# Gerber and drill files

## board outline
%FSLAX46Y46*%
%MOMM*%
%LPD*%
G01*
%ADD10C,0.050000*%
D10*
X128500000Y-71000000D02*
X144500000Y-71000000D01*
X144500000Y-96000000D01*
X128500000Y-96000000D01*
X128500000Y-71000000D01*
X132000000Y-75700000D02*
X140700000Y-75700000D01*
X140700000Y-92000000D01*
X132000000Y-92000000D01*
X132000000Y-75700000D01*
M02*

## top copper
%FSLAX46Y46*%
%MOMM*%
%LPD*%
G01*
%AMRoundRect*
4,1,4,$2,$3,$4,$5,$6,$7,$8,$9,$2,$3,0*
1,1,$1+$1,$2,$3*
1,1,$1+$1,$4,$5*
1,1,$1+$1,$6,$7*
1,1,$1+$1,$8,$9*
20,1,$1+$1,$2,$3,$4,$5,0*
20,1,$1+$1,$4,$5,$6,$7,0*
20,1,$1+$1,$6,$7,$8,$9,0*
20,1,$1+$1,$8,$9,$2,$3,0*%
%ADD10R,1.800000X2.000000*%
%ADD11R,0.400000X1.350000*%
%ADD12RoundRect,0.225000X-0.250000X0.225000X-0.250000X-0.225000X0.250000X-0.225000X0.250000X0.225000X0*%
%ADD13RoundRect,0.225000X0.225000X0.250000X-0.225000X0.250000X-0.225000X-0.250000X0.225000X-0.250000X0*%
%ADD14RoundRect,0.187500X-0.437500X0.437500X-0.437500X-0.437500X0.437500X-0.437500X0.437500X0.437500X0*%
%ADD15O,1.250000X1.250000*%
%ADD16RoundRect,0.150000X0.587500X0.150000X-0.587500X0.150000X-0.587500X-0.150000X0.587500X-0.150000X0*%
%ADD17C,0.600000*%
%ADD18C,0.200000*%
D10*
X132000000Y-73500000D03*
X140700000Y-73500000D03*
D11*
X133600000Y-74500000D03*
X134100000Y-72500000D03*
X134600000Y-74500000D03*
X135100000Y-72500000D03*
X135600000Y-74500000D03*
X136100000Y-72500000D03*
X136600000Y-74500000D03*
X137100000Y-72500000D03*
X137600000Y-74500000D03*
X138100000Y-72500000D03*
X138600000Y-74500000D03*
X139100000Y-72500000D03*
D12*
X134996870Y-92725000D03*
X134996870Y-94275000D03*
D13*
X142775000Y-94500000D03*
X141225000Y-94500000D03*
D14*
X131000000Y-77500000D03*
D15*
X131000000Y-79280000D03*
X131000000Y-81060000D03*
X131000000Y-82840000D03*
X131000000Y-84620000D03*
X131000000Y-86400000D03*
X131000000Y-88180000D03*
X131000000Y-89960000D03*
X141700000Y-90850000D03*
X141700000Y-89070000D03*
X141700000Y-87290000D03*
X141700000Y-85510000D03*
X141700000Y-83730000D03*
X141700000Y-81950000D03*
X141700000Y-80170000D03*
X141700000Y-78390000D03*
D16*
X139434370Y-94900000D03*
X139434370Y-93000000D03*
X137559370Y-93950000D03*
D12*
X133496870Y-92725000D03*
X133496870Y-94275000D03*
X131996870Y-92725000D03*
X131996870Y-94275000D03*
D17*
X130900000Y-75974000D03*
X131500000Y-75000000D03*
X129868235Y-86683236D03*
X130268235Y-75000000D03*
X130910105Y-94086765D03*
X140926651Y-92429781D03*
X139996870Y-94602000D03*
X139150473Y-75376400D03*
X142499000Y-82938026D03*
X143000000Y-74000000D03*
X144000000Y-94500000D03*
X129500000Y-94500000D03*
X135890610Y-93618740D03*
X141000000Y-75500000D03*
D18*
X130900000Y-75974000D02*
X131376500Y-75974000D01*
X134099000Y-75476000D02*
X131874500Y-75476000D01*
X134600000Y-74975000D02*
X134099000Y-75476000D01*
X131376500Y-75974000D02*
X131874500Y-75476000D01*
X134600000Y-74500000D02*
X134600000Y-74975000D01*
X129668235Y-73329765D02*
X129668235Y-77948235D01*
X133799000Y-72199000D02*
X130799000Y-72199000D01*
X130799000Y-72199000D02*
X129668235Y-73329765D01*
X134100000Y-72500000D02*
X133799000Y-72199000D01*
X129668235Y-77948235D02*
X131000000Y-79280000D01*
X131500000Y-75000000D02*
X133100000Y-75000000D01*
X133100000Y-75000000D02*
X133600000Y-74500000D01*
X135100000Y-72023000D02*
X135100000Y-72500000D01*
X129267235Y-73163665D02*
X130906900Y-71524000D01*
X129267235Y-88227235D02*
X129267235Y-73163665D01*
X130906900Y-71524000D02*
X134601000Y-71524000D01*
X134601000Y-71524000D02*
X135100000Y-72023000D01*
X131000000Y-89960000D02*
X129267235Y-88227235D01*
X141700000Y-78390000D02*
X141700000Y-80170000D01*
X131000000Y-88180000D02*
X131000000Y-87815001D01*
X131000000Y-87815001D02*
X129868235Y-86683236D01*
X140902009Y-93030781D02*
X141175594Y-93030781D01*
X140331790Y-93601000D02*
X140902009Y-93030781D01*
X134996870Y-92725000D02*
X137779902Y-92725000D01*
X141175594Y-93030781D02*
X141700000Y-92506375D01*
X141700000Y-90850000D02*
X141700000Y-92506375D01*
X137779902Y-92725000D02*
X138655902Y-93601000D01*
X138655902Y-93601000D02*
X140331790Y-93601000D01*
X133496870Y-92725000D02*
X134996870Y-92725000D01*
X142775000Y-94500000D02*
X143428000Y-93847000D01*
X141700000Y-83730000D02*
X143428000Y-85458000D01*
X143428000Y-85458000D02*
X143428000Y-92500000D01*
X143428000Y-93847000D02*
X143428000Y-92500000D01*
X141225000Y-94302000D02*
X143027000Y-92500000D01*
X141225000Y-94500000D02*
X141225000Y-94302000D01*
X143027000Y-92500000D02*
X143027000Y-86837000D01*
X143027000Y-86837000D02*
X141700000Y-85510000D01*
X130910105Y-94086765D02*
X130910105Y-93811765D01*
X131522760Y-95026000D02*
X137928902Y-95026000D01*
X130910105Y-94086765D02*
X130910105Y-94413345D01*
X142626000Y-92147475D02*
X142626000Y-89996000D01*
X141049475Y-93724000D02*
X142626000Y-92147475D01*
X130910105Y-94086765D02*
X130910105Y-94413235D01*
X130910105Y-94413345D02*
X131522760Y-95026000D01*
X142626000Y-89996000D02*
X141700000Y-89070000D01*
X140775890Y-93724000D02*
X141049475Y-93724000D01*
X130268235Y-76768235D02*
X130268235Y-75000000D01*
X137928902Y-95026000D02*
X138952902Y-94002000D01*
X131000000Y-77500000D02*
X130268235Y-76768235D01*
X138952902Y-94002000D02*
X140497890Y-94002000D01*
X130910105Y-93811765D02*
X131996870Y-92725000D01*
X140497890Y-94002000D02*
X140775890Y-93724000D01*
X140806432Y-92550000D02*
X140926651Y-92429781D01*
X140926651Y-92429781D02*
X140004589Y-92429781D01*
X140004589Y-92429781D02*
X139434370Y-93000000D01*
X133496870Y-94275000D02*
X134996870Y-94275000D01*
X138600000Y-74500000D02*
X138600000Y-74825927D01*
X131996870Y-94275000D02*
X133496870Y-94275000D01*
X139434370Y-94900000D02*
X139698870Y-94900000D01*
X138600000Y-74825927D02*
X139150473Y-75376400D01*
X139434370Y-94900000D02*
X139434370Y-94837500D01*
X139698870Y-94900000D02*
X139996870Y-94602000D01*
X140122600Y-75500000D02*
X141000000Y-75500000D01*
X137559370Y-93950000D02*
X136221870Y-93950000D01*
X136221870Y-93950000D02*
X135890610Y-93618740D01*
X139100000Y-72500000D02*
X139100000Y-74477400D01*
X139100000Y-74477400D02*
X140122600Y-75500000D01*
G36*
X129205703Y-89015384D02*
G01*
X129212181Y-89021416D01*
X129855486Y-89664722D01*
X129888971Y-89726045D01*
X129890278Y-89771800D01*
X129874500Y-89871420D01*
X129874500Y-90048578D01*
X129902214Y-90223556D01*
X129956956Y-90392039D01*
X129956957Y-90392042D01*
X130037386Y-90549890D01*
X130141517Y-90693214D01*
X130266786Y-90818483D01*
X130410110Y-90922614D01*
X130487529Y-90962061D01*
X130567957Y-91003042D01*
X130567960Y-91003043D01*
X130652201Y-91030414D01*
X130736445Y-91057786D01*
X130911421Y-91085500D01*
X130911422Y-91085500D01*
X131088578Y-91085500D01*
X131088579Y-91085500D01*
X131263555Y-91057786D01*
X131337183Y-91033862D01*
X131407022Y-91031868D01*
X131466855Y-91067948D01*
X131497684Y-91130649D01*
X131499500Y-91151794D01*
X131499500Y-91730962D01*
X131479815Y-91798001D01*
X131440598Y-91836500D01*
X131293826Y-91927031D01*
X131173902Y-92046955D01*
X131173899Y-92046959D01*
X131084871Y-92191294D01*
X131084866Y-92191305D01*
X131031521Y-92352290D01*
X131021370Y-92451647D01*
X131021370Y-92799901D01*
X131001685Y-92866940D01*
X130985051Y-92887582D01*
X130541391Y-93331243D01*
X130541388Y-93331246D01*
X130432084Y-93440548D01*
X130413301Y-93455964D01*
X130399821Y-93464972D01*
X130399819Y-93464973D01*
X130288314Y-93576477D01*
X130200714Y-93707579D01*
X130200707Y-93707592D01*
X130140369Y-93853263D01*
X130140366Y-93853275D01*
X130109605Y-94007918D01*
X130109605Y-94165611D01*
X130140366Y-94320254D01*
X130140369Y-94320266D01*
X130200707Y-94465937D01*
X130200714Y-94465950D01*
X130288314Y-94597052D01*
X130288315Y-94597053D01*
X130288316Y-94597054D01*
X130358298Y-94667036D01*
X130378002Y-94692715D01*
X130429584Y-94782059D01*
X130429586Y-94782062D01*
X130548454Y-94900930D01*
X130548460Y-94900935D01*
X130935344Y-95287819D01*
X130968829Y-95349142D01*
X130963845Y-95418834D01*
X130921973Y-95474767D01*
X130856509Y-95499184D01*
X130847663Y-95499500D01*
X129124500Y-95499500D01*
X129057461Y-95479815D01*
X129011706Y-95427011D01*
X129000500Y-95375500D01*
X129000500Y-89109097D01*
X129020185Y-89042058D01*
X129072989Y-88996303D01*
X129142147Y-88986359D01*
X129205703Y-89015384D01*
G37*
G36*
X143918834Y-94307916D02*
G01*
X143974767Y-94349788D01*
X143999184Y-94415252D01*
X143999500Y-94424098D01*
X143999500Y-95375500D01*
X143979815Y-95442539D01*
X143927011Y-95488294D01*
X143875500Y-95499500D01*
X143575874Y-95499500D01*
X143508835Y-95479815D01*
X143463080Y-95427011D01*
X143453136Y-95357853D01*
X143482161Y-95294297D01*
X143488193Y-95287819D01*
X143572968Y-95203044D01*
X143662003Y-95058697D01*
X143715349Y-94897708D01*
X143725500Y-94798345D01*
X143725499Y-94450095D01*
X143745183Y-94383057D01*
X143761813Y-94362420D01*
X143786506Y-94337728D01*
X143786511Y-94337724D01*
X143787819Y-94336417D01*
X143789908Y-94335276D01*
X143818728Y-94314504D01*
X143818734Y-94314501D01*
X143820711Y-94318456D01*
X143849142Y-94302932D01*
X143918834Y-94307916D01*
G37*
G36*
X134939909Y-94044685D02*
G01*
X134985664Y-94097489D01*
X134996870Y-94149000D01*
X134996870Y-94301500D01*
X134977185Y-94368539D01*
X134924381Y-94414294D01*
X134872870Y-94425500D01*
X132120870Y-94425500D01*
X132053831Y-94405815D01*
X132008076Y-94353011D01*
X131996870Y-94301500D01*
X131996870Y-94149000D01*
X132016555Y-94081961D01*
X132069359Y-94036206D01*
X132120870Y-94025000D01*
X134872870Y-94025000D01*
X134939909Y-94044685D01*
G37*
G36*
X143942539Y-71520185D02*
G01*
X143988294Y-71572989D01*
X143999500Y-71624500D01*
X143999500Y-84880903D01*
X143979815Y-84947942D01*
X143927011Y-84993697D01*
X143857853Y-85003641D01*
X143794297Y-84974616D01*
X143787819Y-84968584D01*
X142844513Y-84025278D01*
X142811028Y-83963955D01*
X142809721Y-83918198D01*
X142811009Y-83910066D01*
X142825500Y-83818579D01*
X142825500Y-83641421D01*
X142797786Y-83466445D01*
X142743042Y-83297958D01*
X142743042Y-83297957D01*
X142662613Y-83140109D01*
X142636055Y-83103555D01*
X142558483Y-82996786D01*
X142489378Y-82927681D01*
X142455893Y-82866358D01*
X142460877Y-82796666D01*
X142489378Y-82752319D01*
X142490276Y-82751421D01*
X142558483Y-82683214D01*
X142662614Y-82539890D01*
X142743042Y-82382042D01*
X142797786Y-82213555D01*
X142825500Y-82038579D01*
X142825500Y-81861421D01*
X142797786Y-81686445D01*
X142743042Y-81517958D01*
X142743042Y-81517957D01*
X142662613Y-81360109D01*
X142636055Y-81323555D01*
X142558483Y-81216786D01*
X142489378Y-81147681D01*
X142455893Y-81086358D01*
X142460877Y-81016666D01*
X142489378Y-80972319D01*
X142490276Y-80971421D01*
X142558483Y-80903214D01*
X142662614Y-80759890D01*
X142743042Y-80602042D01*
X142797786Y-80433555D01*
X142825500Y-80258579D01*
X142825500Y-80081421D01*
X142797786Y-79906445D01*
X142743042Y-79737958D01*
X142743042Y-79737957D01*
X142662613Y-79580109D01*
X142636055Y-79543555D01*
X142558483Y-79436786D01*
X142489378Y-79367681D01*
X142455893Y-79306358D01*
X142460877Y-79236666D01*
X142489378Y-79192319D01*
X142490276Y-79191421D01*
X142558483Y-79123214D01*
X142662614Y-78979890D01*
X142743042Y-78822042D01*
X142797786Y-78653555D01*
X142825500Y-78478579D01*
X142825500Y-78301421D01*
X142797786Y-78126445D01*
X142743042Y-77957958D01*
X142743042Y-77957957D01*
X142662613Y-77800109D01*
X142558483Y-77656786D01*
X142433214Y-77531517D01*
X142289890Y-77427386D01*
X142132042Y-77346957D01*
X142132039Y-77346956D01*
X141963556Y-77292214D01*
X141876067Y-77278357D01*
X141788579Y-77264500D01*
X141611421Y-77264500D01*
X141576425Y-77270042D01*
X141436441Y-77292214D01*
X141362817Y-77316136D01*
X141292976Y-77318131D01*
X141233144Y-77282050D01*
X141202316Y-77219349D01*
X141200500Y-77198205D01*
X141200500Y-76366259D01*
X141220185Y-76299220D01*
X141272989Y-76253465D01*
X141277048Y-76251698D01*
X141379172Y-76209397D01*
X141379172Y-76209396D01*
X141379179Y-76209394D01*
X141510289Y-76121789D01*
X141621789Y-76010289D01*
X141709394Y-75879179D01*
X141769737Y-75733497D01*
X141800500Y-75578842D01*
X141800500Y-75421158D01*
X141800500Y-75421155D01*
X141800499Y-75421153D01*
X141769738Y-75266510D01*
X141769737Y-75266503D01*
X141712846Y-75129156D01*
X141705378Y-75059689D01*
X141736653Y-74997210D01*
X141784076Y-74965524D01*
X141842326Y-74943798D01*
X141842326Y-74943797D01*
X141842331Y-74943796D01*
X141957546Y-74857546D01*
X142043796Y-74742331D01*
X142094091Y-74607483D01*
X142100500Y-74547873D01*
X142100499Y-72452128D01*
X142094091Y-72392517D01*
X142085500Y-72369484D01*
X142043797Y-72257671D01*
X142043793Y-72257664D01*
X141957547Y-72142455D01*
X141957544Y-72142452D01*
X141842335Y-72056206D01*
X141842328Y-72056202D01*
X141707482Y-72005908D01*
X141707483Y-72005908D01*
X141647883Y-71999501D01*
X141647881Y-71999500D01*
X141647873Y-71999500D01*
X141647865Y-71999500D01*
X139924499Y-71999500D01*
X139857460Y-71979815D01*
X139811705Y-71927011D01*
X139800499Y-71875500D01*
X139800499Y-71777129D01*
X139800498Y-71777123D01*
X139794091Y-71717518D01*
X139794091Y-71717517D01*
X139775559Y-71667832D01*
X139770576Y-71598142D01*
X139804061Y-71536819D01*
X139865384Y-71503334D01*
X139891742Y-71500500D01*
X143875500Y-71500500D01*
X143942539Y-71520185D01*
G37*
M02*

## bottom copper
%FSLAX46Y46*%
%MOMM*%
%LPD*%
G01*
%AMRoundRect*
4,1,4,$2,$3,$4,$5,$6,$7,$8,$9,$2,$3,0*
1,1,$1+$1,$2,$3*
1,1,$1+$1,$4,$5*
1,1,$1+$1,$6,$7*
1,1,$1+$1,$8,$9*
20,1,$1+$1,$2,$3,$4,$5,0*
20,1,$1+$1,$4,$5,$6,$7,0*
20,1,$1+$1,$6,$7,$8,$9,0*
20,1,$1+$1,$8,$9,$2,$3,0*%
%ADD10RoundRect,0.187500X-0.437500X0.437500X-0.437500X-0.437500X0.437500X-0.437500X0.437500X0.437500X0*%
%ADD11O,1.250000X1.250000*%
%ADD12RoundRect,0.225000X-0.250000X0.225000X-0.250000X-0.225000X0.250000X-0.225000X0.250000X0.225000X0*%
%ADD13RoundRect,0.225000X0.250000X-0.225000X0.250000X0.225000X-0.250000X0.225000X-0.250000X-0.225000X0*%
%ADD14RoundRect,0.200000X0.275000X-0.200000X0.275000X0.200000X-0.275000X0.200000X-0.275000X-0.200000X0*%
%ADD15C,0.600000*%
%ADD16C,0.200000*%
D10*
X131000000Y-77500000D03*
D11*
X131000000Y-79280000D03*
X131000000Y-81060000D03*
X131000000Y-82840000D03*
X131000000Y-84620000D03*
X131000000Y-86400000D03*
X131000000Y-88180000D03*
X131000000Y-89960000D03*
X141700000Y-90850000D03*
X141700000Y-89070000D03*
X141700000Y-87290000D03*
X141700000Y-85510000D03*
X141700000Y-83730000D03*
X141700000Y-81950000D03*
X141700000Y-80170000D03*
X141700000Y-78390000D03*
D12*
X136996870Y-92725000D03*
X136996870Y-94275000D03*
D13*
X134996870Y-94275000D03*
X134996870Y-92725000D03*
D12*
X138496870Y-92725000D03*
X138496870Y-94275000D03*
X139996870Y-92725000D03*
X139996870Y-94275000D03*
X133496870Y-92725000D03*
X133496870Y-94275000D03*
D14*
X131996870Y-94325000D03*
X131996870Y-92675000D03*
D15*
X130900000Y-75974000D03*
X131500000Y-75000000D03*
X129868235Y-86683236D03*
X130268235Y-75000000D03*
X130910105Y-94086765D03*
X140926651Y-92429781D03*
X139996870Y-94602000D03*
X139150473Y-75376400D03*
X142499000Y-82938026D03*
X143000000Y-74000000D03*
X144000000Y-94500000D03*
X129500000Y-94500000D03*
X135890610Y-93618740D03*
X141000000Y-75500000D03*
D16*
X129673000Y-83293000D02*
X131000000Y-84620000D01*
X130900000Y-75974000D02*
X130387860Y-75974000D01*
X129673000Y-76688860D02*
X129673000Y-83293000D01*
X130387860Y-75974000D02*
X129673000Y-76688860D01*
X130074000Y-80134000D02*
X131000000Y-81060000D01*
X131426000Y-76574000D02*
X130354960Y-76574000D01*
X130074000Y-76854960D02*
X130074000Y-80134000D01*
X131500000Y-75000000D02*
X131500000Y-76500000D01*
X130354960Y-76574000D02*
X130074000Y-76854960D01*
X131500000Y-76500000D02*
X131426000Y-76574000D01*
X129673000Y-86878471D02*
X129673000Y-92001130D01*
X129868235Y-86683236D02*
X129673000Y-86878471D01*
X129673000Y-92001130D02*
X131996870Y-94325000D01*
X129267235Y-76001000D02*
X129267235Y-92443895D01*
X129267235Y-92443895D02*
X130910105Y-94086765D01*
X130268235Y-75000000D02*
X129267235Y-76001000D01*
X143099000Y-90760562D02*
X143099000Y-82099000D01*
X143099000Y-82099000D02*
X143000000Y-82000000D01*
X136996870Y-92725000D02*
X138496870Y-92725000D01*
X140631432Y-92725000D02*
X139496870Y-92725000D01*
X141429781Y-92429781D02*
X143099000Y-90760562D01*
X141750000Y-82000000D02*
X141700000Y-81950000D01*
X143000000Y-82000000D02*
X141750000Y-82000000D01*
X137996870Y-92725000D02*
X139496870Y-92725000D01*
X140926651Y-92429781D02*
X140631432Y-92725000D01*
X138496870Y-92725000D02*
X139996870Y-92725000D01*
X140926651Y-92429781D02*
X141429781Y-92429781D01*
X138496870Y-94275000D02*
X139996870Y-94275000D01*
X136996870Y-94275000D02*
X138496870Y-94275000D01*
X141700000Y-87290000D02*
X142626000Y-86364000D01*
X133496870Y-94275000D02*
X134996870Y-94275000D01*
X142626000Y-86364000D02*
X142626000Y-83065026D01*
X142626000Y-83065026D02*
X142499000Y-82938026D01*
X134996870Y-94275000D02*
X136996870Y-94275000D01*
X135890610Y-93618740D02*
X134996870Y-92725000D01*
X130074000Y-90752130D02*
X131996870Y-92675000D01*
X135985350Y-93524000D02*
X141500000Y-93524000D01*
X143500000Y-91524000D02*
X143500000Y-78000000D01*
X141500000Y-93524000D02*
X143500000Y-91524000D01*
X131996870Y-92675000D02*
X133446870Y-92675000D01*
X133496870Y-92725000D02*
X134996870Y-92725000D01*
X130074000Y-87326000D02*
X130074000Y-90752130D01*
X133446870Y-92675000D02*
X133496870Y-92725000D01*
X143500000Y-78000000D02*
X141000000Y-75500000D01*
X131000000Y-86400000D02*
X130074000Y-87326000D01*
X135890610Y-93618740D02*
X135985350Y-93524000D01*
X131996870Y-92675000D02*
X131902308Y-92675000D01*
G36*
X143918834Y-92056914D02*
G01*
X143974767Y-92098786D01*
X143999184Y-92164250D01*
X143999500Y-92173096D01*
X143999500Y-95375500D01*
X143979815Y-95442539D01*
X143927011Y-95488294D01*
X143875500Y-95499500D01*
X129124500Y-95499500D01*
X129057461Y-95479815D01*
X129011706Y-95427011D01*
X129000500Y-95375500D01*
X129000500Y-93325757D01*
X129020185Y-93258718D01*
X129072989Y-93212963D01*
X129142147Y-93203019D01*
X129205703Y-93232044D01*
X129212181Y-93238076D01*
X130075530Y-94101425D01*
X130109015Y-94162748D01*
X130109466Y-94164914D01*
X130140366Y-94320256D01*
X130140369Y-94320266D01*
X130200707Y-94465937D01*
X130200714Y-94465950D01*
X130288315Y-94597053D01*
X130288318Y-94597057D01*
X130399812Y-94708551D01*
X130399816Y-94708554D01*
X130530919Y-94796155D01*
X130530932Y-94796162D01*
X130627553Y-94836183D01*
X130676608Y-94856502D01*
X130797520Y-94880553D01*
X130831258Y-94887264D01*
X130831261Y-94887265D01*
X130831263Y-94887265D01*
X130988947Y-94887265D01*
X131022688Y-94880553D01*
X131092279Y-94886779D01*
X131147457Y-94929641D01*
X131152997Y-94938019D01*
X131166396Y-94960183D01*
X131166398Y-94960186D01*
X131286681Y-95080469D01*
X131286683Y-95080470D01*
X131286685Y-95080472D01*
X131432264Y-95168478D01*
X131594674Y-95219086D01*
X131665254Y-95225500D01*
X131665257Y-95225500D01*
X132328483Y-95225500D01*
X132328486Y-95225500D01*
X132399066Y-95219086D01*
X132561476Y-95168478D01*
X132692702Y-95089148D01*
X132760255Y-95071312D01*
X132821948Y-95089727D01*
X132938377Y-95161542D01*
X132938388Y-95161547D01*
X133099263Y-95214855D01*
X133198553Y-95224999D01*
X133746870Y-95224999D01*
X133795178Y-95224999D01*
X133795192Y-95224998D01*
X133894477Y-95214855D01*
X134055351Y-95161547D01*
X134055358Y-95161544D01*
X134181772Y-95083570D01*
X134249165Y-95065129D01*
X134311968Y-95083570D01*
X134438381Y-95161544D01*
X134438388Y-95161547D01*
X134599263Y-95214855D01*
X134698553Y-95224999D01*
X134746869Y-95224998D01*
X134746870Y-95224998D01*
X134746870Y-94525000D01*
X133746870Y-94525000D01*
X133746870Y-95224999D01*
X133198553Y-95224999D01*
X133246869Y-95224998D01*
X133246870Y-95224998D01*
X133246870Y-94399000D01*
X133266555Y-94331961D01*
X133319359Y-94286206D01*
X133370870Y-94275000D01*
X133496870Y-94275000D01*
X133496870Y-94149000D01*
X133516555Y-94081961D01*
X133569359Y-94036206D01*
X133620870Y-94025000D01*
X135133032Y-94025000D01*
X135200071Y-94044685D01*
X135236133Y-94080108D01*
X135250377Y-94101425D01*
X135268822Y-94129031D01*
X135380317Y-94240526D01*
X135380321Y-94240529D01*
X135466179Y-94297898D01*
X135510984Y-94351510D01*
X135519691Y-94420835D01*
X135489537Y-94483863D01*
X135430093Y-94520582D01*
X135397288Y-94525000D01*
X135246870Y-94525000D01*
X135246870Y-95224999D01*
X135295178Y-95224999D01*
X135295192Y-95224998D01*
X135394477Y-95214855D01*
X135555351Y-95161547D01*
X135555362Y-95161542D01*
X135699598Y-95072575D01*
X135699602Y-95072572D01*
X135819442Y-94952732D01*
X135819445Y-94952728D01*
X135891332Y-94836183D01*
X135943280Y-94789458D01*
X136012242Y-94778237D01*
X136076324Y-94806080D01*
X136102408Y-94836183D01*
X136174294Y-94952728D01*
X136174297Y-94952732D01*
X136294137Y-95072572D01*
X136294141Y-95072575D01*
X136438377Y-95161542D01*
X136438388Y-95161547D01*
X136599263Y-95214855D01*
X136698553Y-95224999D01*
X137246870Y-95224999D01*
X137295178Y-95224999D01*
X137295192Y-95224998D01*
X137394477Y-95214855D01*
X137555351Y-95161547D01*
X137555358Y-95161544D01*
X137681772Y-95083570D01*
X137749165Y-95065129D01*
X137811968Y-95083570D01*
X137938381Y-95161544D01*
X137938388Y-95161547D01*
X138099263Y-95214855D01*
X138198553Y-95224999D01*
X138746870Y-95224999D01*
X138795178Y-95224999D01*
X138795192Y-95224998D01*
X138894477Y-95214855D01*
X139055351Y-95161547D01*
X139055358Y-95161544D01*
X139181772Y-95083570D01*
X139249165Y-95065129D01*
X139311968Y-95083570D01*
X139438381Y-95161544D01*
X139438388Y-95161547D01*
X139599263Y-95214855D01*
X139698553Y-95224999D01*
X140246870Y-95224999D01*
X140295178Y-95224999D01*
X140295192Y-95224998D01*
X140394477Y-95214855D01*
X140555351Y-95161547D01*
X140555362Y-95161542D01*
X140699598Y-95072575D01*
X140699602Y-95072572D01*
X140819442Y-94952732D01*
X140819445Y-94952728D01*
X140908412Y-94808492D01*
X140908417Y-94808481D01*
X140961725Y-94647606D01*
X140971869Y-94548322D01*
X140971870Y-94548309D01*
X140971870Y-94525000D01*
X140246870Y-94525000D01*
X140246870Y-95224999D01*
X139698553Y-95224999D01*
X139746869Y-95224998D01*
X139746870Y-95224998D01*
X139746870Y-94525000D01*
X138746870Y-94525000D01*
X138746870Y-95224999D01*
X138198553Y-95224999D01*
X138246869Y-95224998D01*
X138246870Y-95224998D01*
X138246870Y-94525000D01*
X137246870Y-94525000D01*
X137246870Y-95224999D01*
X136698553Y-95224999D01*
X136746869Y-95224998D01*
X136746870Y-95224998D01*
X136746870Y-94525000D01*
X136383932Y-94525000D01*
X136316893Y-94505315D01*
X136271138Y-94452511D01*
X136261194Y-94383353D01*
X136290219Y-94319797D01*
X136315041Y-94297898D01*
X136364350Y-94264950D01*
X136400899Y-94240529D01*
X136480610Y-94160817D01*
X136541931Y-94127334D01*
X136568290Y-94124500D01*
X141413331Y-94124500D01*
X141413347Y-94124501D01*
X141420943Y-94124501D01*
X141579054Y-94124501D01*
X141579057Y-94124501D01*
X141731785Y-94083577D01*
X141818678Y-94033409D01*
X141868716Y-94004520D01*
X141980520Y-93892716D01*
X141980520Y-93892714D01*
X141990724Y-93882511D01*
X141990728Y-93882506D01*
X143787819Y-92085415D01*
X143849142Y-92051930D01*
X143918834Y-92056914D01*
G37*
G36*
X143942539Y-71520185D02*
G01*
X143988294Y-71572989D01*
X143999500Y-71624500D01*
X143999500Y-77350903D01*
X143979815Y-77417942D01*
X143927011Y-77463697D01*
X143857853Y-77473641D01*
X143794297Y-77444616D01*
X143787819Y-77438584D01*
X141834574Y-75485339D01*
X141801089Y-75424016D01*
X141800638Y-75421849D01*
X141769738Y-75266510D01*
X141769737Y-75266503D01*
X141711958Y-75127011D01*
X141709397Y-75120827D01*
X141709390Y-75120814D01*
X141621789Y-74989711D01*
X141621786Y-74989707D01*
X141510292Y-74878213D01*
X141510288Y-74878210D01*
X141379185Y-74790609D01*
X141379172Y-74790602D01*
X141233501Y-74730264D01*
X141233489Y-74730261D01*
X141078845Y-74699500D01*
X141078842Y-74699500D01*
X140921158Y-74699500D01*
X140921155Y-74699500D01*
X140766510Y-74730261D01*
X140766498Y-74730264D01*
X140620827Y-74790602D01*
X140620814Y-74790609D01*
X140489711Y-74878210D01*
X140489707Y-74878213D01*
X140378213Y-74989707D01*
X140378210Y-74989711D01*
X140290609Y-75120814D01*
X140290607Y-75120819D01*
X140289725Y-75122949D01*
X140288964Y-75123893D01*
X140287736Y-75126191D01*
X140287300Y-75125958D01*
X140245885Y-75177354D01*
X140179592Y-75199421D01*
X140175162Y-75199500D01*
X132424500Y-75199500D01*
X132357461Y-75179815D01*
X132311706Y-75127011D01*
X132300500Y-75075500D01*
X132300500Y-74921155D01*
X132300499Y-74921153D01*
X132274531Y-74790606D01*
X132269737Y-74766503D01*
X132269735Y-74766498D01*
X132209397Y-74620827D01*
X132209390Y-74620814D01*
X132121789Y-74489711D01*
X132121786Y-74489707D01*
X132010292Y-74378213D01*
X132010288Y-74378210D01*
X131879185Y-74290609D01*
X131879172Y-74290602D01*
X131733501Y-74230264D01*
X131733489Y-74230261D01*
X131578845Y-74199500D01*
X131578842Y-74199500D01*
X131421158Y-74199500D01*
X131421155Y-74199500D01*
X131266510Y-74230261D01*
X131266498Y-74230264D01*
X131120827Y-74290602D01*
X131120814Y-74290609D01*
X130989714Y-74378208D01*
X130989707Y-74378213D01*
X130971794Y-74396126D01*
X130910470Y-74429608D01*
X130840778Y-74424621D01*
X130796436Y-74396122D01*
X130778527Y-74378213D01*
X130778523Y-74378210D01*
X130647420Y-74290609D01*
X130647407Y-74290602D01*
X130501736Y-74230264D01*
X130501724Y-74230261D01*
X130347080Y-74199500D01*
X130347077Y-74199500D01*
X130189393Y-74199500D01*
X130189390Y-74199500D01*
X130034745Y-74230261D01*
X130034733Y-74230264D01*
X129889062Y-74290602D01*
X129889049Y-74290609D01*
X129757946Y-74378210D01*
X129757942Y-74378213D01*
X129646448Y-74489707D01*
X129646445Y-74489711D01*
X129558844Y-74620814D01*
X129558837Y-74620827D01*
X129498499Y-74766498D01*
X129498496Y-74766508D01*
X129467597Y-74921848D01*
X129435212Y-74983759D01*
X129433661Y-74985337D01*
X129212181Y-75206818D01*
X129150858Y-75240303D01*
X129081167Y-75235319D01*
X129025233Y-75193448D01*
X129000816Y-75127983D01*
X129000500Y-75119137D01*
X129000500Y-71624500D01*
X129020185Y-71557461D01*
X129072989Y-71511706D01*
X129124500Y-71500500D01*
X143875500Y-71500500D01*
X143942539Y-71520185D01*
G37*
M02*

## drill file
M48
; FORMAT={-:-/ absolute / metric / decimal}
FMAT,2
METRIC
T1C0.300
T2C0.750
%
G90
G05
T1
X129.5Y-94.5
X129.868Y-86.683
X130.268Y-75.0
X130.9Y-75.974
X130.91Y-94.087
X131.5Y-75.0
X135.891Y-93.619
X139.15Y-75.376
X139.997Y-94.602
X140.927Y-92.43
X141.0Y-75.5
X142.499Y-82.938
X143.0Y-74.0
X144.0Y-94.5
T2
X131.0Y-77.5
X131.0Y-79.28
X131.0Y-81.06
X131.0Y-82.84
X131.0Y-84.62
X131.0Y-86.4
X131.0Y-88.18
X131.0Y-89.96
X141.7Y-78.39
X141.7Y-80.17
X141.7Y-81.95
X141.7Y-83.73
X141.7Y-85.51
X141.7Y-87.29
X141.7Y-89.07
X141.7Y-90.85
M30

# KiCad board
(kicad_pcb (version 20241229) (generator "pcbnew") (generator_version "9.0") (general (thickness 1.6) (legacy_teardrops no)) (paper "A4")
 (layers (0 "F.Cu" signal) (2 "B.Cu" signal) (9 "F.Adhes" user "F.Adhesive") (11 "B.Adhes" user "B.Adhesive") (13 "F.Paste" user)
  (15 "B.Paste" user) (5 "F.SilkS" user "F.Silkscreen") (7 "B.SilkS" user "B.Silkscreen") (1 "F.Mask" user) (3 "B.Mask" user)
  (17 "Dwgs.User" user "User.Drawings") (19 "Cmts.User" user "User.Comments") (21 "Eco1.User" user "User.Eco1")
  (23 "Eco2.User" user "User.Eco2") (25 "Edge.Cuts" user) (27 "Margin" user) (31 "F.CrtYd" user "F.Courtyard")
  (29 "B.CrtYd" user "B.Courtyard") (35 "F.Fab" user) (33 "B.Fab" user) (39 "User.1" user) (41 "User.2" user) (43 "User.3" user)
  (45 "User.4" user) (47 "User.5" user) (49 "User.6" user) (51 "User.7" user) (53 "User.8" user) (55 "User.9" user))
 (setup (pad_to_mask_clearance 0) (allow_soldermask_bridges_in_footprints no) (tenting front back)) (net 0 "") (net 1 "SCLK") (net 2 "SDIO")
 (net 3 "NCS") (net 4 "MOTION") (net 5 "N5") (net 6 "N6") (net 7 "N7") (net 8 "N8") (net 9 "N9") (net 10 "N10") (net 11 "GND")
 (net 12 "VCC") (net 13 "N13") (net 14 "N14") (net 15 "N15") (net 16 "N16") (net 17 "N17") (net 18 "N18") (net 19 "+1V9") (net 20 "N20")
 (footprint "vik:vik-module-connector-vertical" (layer "F.Cu") (at 136.35 73.5)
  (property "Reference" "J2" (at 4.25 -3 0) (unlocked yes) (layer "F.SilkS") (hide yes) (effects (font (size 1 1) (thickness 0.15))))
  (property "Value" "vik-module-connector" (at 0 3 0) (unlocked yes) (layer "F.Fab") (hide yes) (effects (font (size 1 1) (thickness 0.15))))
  (pad "" smd rect (at -4.35 0) (size 1.8 2) (layers "F.Cu" "F.Mask" "F.Paste") (thermal_bridge_angle 45))
  (pad "" smd rect (at 4.35 0) (size 1.8 2) (layers "F.Cu" "F.Mask" "F.Paste") (thermal_bridge_angle 45))
  (pad "1" smd rect (at -2.75 1) (size 0.4 1.35) (layers "F.Cu" "F.Mask" "F.Paste") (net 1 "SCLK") (thermal_bridge_angle 45))
  (pad "2" smd rect (at -2.25 -1) (size 0.4 1.35) (layers "F.Cu" "F.Mask" "F.Paste") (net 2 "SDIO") (thermal_bridge_angle 45))
  (pad "3" smd rect (at -1.75 1) (size 0.4 1.35) (layers "F.Cu" "F.Mask" "F.Paste") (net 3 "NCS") (thermal_bridge_angle 45))
  (pad "4" smd rect (at -1.25 -1) (size 0.4 1.35) (layers "F.Cu" "F.Mask" "F.Paste") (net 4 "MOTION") (thermal_bridge_angle 45))
  (pad "5" smd rect (at -0.75 1) (size 0.4 1.35) (layers "F.Cu" "F.Mask" "F.Paste") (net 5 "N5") (thermal_bridge_angle 45))
  (pad "6" smd rect (at -0.25 -1) (size 0.4 1.35) (layers "F.Cu" "F.Mask" "F.Paste") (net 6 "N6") (thermal_bridge_angle 45))
  (pad "7" smd rect (at 0.25 1) (size 0.4 1.35) (layers "F.Cu" "F.Mask" "F.Paste") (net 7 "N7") (thermal_bridge_angle 45))
  (pad "8" smd rect (at 0.75 -1) (size 0.4 1.35) (layers "F.Cu" "F.Mask" "F.Paste") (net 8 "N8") (thermal_bridge_angle 45))
  (pad "9" smd rect (at 1.25 1) (size 0.4 1.35) (layers "F.Cu" "F.Mask" "F.Paste") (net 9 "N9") (thermal_bridge_angle 45))
  (pad "10" smd rect (at 1.75 -1) (size 0.4 1.35) (layers "F.Cu" "F.Mask" "F.Paste") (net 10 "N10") (thermal_bridge_angle 45))
  (pad "11" smd rect (at 2.25 1) (size 0.4 1.35) (layers "F.Cu" "F.Mask" "F.Paste") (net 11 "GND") (thermal_bridge_angle 45))
  (pad "12" smd rect (at 2.75 -1) (size 0.4 1.35) (layers "F.Cu" "F.Mask" "F.Paste") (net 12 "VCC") (thermal_bridge_angle 45)))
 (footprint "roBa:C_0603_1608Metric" (layer "F.Cu") (at 134.99687 93.5 -90)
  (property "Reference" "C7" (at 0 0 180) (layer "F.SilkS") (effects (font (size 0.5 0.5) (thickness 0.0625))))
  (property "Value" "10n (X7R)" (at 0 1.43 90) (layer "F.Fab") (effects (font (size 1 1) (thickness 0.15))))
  (pad "1" smd roundrect (at -0.775 0 270) (size 0.9 0.95) (layers "F.Cu" "F.Mask" "F.Paste") (roundrect_rratio 0.25) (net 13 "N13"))
  (pad "2" smd roundrect (at 0.775 0 270) (size 0.9 0.95) (layers "F.Cu" "F.Mask" "F.Paste") (roundrect_rratio 0.25) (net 11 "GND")))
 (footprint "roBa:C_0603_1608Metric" (layer "F.Cu") (at 142 94.5 180)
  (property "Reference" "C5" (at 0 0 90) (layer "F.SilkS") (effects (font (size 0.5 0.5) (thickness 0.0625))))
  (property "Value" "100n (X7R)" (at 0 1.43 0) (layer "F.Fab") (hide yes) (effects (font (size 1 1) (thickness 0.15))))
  (pad "1" smd roundrect (at -0.775 0 180) (size 0.9 0.95) (layers "F.Cu" "F.Mask" "F.Paste") (roundrect_rratio 0.25) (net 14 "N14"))
  (pad "2" smd roundrect (at 0.775 0 180) (size 0.9 0.95) (layers "F.Cu" "F.Mask" "F.Paste") (roundrect_rratio 0.25) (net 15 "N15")))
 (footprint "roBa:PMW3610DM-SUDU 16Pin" (layer "F.Cu") (at 136.35 83.668 90)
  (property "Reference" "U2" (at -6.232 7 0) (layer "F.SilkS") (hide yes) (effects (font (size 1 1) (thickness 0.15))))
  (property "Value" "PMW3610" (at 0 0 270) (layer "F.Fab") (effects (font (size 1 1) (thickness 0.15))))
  (pad "1" thru_hole roundrect (at 6.168 -5.35 270) (size 1.25 1.25) (drill 0.75) (layers "*.Cu" "*.Mask") (remove_unused_layers no)
   (roundrect_rratio 0.15) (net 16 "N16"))
  (pad "2" thru_hole oval (at 4.388 -5.35 270) (size 1.25 1.25) (drill 0.75) (layers "*.Cu" "*.Mask") (remove_unused_layers no)
   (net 2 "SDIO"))
  (pad "3" thru_hole oval (at 2.608 -5.35 270) (size 1.25 1.25) (drill 0.75) (layers "*.Cu" "*.Mask") (remove_unused_layers no)
   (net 1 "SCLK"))
  (pad "4" thru_hole oval (at 0.828 -5.35 270) (size 1.25 1.25) (drill 0.75) (layers "*.Cu" "*.Mask") (remove_unused_layers no)
   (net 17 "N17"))
  (pad "5" thru_hole oval (at -0.952 -5.35 270) (size 1.25 1.25) (drill 0.75) (layers "*.Cu" "*.Mask") (remove_unused_layers no)
   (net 3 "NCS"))
  (pad "6" thru_hole oval (at -2.732 -5.35 270) (size 1.25 1.25) (drill 0.75) (layers "*.Cu" "*.Mask") (remove_unused_layers no)
   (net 12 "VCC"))
  (pad "7" thru_hole oval (at -4.512 -5.35 270) (size 1.25 1.25) (drill 0.75) (layers "*.Cu" "*.Mask") (remove_unused_layers no)
   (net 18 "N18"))
  (pad "8" thru_hole oval (at -6.292 -5.35 270) (size 1.25 1.25) (drill 0.75) (layers "*.Cu" "*.Mask") (remove_unused_layers no)
   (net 4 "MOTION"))
  (pad "9" thru_hole oval (at -7.182 5.35 270) (size 1.25 1.25) (drill 0.75) (layers "*.Cu" "*.Mask") (remove_unused_layers no)
   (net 13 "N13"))
  (pad "10" thru_hole oval (at -5.402 5.35 270) (size 1.25 1.25) (drill 0.75) (layers "*.Cu" "*.Mask") (remove_unused_layers no)
   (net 16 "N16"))
  (pad "11" thru_hole oval (at -3.622 5.35 270) (size 1.25 1.25) (drill 0.75) (layers "*.Cu" "*.Mask") (remove_unused_layers no)
   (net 11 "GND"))
  (pad "12" thru_hole oval (at -1.842 5.35 270) (size 1.25 1.25) (drill 0.75) (layers "*.Cu" "*.Mask") (remove_unused_layers no)
   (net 15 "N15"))
  (pad "13" thru_hole oval (at -0.062 5.35 270) (size 1.25 1.25) (drill 0.75) (layers "*.Cu" "*.Mask") (remove_unused_layers no)
   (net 14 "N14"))
  (pad "14" thru_hole oval (at 1.718 5.35 270) (size 1.25 1.25) (drill 0.75) (layers "*.Cu" "*.Mask") (remove_unused_layers no)
   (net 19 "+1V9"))
  (pad "15" thru_hole oval (at 3.498 5.35 270) (size 1.25 1.25) (drill 0.75) (layers "*.Cu" "*.Mask") (remove_unused_layers no)
   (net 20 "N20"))
  (pad "16" thru_hole oval (at 5.278 5.35 270) (size 1.25 1.25) (drill 0.75) (layers "*.Cu" "*.Mask") (remove_unused_layers no)
   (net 20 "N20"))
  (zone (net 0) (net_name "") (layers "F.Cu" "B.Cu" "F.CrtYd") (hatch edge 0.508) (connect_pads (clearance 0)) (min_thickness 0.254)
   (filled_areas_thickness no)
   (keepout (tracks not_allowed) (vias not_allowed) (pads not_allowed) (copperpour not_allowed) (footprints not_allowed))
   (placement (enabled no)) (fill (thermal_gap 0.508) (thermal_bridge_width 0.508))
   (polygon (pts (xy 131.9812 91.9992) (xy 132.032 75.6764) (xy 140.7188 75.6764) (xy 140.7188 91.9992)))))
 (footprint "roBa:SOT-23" (layer "F.Cu") (at 138.49687 93.95 180)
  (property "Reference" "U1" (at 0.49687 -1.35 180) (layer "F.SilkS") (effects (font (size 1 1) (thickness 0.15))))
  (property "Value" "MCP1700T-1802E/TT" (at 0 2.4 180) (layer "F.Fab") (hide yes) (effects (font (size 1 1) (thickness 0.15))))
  (pad "1" smd roundrect (at -0.9375 -0.95 180) (size 1.475 0.6) (layers "F.Cu" "F.Mask" "F.Paste") (roundrect_rratio 0.25) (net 11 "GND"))
  (pad "2" smd roundrect (at -0.9375 0.95 180) (size 1.475 0.6) (layers "F.Cu" "F.Mask" "F.Paste") (roundrect_rratio 0.25) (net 19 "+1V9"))
  (pad "3" smd roundrect (at 0.9375 0 180) (size 1.475 0.6) (layers "F.Cu" "F.Mask" "F.Paste") (roundrect_rratio 0.25) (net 12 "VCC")))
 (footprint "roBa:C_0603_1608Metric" (layer "F.Cu") (at 133.49687 93.5 -90)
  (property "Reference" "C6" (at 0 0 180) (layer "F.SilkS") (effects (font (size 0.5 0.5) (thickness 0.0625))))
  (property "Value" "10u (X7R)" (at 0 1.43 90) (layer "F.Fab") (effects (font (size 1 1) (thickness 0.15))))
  (pad "1" smd roundrect (at -0.775 0 270) (size 0.9 0.95) (layers "F.Cu" "F.Mask" "F.Paste") (roundrect_rratio 0.25) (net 13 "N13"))
  (pad "2" smd roundrect (at 0.775 0 270) (size 0.9 0.95) (layers "F.Cu" "F.Mask" "F.Paste") (roundrect_rratio 0.25) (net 11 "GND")))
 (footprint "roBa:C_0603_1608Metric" (layer "F.Cu") (at 131.99687 93.5 -90)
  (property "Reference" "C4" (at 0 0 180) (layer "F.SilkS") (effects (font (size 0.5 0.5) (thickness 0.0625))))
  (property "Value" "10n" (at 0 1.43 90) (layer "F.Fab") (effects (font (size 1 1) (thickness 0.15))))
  (pad "1" smd roundrect (at -0.775 0 270) (size 0.9 0.95) (layers "F.Cu" "F.Mask" "F.Paste") (roundrect_rratio 0.25) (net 16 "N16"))
  (pad "2" smd roundrect (at 0.775 0 270) (size 0.9 0.95) (layers "F.Cu" "F.Mask" "F.Paste") (roundrect_rratio 0.25) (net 11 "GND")))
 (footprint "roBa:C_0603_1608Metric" (layer "B.Cu") (at 136.99687 93.5 -90)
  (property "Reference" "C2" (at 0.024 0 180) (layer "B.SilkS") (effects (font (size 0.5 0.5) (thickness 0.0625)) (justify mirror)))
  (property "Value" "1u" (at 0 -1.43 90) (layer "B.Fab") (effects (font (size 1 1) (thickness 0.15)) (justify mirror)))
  (pad "1" smd roundrect (at -0.775 0 270) (size 0.9 0.95) (layers "B.Cu" "B.Mask" "B.Paste") (roundrect_rratio 0.25) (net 19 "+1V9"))
  (pad "2" smd roundrect (at 0.775 0 270) (size 0.9 0.95) (layers "B.Cu" "B.Mask" "B.Paste") (roundrect_rratio 0.25) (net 11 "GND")))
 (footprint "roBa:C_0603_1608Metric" (layer "B.Cu") (at 134.99687 93.5 90)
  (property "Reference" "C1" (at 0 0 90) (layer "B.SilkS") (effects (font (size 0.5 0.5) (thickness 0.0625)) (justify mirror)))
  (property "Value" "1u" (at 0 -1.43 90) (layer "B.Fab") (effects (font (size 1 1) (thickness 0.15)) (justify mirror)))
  (pad "1" smd roundrect (at -0.775 0 90) (size 0.9 0.95) (layers "B.Cu" "B.Mask" "B.Paste") (roundrect_rratio 0.25) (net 11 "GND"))
  (pad "2" smd roundrect (at 0.775 0 90) (size 0.9 0.95) (layers "B.Cu" "B.Mask" "B.Paste") (roundrect_rratio 0.25) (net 12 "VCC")))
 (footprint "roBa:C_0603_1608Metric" (layer "B.Cu") (at 138.49687 93.5 -90)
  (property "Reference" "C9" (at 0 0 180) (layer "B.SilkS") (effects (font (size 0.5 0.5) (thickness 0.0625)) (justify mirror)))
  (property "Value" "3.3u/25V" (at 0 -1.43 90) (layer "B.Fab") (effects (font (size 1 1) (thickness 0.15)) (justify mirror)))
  (pad "1" smd roundrect (at -0.775 0 270) (size 0.9 0.95) (layers "B.Cu" "B.Mask" "B.Paste") (roundrect_rratio 0.25) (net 19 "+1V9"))
  (pad "2" smd roundrect (at 0.775 0 270) (size 0.9 0.95) (layers "B.Cu" "B.Mask" "B.Paste") (roundrect_rratio 0.25) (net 11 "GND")))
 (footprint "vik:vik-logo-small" (layer "B.Cu") (at 142 74 90)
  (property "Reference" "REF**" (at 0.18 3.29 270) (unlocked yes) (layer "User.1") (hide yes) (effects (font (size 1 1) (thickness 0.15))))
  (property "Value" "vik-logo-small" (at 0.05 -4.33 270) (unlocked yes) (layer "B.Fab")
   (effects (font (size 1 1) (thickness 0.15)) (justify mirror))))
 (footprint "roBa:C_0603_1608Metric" (layer "B.Cu") (at 139.99687 93.5 -90)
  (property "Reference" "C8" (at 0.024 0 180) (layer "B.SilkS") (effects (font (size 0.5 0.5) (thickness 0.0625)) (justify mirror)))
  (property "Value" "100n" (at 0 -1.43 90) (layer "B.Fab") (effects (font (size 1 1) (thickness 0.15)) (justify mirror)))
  (pad "1" smd roundrect (at -0.775 0 270) (size 0.9 0.95) (layers "B.Cu" "B.Mask" "B.Paste") (roundrect_rratio 0.25) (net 19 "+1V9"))
  (pad "2" smd roundrect (at 0.775 0 270) (size 0.9 0.95) (layers "B.Cu" "B.Mask" "B.Paste") (roundrect_rratio 0.25) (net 11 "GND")))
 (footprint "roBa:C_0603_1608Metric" (layer "B.Cu") (at 133.49687 93.5 -90)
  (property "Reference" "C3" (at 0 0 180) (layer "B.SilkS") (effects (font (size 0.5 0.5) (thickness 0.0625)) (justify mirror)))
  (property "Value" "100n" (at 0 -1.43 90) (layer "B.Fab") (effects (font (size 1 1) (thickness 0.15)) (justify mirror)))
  (pad "1" smd roundrect (at -0.775 0 270) (size 0.9 0.95) (layers "B.Cu" "B.Mask" "B.Paste") (roundrect_rratio 0.25) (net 12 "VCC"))
  (pad "2" smd roundrect (at 0.775 0 270) (size 0.9 0.95) (layers "B.Cu" "B.Mask" "B.Paste") (roundrect_rratio 0.25) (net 11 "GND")))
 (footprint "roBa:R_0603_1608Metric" (layer "B.Cu") (at 131.99687 93.5 90)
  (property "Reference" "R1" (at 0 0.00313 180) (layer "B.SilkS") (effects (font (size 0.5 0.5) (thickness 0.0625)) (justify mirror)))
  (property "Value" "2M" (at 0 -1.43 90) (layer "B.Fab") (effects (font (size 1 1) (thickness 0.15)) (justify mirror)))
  (pad "1" smd roundrect (at -0.825 0 90) (size 0.8 0.95) (layers "B.Cu" "B.Mask" "B.Paste") (roundrect_rratio 0.25) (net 18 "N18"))
  (pad "2" smd roundrect (at 0.825 0 90) (size 0.8 0.95) (layers "B.Cu" "B.Mask" "B.Paste") (roundrect_rratio 0.25) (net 12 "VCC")))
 (gr_rect (start 128.5 71) (end 144.5 96) (stroke (width 0.05) (type default)) (fill no) (layer "Edge.Cuts"))
 (gr_rect (start 132 75.7) (end 140.7 92) (stroke (width 0.05) (type default)) (fill no) (layer "Edge.Cuts"))
 (segment (start 130.9 75.974) (end 131.3765 75.974) (width 0.2) (layer "F.Cu") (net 3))
 (segment (start 134.099 75.476) (end 131.8745 75.476) (width 0.2) (layer "F.Cu") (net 3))
 (segment (start 134.6 74.975) (end 134.099 75.476) (width 0.2) (layer "F.Cu") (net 3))
 (segment (start 131.3765 75.974) (end 131.8745 75.476) (width 0.2) (layer "F.Cu") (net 3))
 (segment (start 134.6 74.5) (end 134.6 74.975) (width 0.2) (layer "F.Cu") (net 3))
 (via (at 130.9 75.974) (size 0.6) (drill 0.3) (layers "F.Cu" "B.Cu") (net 3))
 (segment (start 129.673 83.293) (end 131 84.62) (width 0.2) (layer "B.Cu") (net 3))
 (segment (start 130.9 75.974) (end 130.38786 75.974) (width 0.2) (layer "B.Cu") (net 3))
 (segment (start 129.673 76.68886) (end 129.673 83.293) (width 0.2) (layer "B.Cu") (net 3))
 (segment (start 130.38786 75.974) (end 129.673 76.68886) (width 0.2) (layer "B.Cu") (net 3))
 (segment (start 129.668235 73.329765) (end 129.668235 77.948235) (width 0.2) (layer "F.Cu") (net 2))
 (segment (start 133.799 72.199) (end 130.799 72.199) (width 0.2) (layer "F.Cu") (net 2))
 (segment (start 130.799 72.199) (end 129.668235 73.329765) (width 0.2) (layer "F.Cu") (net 2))
 (segment (start 134.1 72.5) (end 133.799 72.199) (width 0.2) (layer "F.Cu") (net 2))
 (segment (start 129.668235 77.948235) (end 131 79.28) (width 0.2) (layer "F.Cu") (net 2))
 (segment (start 131.5 75) (end 133.1 75) (width 0.2) (layer "F.Cu") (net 1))
 (segment (start 133.1 75) (end 133.6 74.5) (width 0.2) (layer "F.Cu") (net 1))
 (via (at 131.5 75) (size 0.6) (drill 0.3) (layers "F.Cu" "B.Cu") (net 1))
 (segment (start 130.074 80.134) (end 131 81.06) (width 0.2) (layer "B.Cu") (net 1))
 (segment (start 131.426 76.574) (end 130.35496 76.574) (width 0.2) (layer "B.Cu") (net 1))
 (segment (start 130.074 76.85496) (end 130.074 80.134) (width 0.2) (layer "B.Cu") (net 1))
 (segment (start 131.5 75) (end 131.5 76.5) (width 0.2) (layer "B.Cu") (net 1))
 (segment (start 130.35496 76.574) (end 130.074 76.85496) (width 0.2) (layer "B.Cu") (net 1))
 (segment (start 131.5 76.5) (end 131.426 76.574) (width 0.2) (layer "B.Cu") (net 1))
 (segment (start 135.1 72.023) (end 135.1 72.5) (width 0.2) (layer "F.Cu") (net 4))
 (segment (start 129.267235 73.163665) (end 130.9069 71.524) (width 0.2) (layer "F.Cu") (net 4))
 (segment (start 129.267235 88.227235) (end 129.267235 73.163665) (width 0.2) (layer "F.Cu") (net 4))
 (segment (start 130.9069 71.524) (end 134.601 71.524) (width 0.2) (layer "F.Cu") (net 4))
 (segment (start 134.601 71.524) (end 135.1 72.023) (width 0.2) (layer "F.Cu") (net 4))
 (segment (start 131 89.96) (end 129.267235 88.227235) (width 0.2) (layer "F.Cu") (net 4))
 (segment (start 141.7 78.39) (end 141.7 80.17) (width 0.2) (layer "F.Cu") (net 20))
 (segment (start 131 88.18) (end 131 87.815001) (width 0.2) (layer "F.Cu") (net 18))
 (segment (start 131 87.815001) (end 129.868235 86.683236) (width 0.2) (layer "F.Cu") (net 18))
 (via (at 129.868235 86.683236) (size 0.6) (drill 0.3) (layers "F.Cu" "B.Cu") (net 18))
 (segment (start 129.673 86.878471) (end 129.673 92.00113) (width 0.2) (layer "B.Cu") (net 18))
 (segment (start 129.868235 86.683236) (end 129.673 86.878471) (width 0.2) (layer "B.Cu") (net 18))
 (segment (start 129.673 92.00113) (end 131.99687 94.325) (width 0.2) (layer "B.Cu") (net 18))
 (segment (start 140.902009 93.030781) (end 141.175594 93.030781) (width 0.2) (layer "F.Cu") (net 13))
 (segment (start 140.33179 93.601) (end 140.902009 93.030781) (width 0.2) (layer "F.Cu") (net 13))
 (segment (start 134.99687 92.725) (end 137.779902 92.725) (width 0.2) (layer "F.Cu") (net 13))
 (segment (start 141.175594 93.030781) (end 141.7 92.506375) (width 0.2) (layer "F.Cu") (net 13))
 (segment (start 141.7 90.85) (end 141.7 92.506375) (width 0.2) (layer "F.Cu") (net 13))
 (segment (start 137.779902 92.725) (end 138.655902 93.601) (width 0.2) (layer "F.Cu") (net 13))
 (segment (start 138.655902 93.601) (end 140.33179 93.601) (width 0.2) (layer "F.Cu") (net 13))
 (segment (start 133.49687 92.725) (end 134.99687 92.725) (width 0.2) (layer "F.Cu") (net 13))
 (segment (start 142.775 94.5) (end 143.428 93.847) (width 0.2) (layer "F.Cu") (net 14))
 (segment (start 141.7 83.73) (end 143.428 85.458) (width 0.2) (layer "F.Cu") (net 14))
 (segment (start 143.428 85.458) (end 143.428 92.5) (width 0.2) (layer "F.Cu") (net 14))
 (segment (start 143.428 93.847) (end 143.428 92.5) (width 0.2) (layer "F.Cu") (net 14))
 (segment (start 141.225 94.302) (end 143.027 92.5) (width 0.2) (layer "F.Cu") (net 15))
 (segment (start 141.225 94.5) (end 141.225 94.302) (width 0.2) (layer "F.Cu") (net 15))
 (segment (start 143.027 92.5) (end 143.027 86.837) (width 0.2) (layer "F.Cu") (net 15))
 (segment (start 143.027 86.837) (end 141.7 85.51) (width 0.2) (layer "F.Cu") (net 15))
 (segment (start 130.910105 94.086765) (end 130.910105 93.811765) (width 0.2) (layer "F.Cu") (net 16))
 (segment (start 131.52276 95.026) (end 137.928902 95.026) (width 0.2) (layer "F.Cu") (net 16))
 (segment (start 130.910105 94.086765) (end 130.910105 94.413345) (width 0.2) (layer "F.Cu") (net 16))
 (segment (start 142.626 92.147475) (end 142.626 89.996) (width 0.2) (layer "F.Cu") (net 16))
 (segment (start 141.049475 93.724) (end 142.626 92.147475) (width 0.2) (layer "F.Cu") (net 16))
 (segment (start 130.910105 94.086765) (end 130.910105 94.413235) (width 0.2) (layer "F.Cu") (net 16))
 (segment (start 130.910105 94.413345) (end 131.52276 95.026) (width 0.2) (layer "F.Cu") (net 16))
 (segment (start 142.626 89.996) (end 141.7 89.07) (width 0.2) (layer "F.Cu") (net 16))
 (segment (start 140.77589 93.724) (end 141.049475 93.724) (width 0.2) (layer "F.Cu") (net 16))
 (segment (start 130.268235 76.768235) (end 130.268235 75) (width 0.2) (layer "F.Cu") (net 16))
 (segment (start 137.928902 95.026) (end 138.952902 94.002) (width 0.2) (layer "F.Cu") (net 16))
 (segment (start 131 77.5) (end 130.268235 76.768235) (width 0.2) (layer "F.Cu") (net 16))
 (segment (start 138.952902 94.002) (end 140.49789 94.002) (width 0.2) (layer "F.Cu") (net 16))
 (segment (start 130.910105 93.811765) (end 131.99687 92.725) (width 0.2) (layer "F.Cu") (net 16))
 (segment (start 140.49789 94.002) (end 140.77589 93.724) (width 0.2) (layer "F.Cu") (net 16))
 (via (at 130.268235 75) (size 0.6) (drill 0.3) (layers "F.Cu" "B.Cu") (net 16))
 (via (at 130.910105 94.086765) (size 0.6) (drill 0.3) (layers "F.Cu" "B.Cu") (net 16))
 (segment (start 129.267235 76.001) (end 129.267235 92.443895) (width 0.2) (layer "B.Cu") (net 16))
 (segment (start 129.267235 92.443895) (end 130.910105 94.086765) (width 0.2) (layer "B.Cu") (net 16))
 (segment (start 130.268235 75) (end 129.267235 76.001) (width 0.2) (layer "B.Cu") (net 16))
 (segment (start 140.806432 92.55) (end 140.926651 92.429781) (width 0.2) (layer "F.Cu") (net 19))
 (segment (start 140.926651 92.429781) (end 140.004589 92.429781) (width 0.2) (layer "F.Cu") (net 19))
 (segment (start 140.004589 92.429781) (end 139.43437 93) (width 0.2) (layer "F.Cu") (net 19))
 (via (at 140.926651 92.429781) (size 0.6) (drill 0.3) (layers "F.Cu" "B.Cu") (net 19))
 (segment (start 143.099 90.760562) (end 143.099 82.099) (width 0.2) (layer "B.Cu") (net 19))
 (segment (start 143.099 82.099) (end 143 82) (width 0.2) (layer "B.Cu") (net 19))
 (segment (start 136.99687 92.725) (end 138.49687 92.725) (width 0.2) (layer "B.Cu") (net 19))
 (segment (start 140.631432 92.725) (end 139.49687 92.725) (width 0.2) (layer "B.Cu") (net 19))
 (segment (start 141.429781 92.429781) (end 143.099 90.760562) (width 0.2) (layer "B.Cu") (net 19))
 (segment (start 141.75 82) (end 141.7 81.95) (width 0.2) (layer "B.Cu") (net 19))
 (segment (start 143 82) (end 141.75 82) (width 0.2) (layer "B.Cu") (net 19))
 (segment (start 137.99687 92.725) (end 139.49687 92.725) (width 0.2) (layer "B.Cu") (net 19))
 (segment (start 140.926651 92.429781) (end 140.631432 92.725) (width 0.2) (layer "B.Cu") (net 19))
 (segment (start 138.49687 92.725) (end 139.99687 92.725) (width 0.2) (layer "B.Cu") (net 19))
 (segment (start 140.926651 92.429781) (end 141.429781 92.429781) (width 0.2) (layer "B.Cu") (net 19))
 (segment (start 133.49687 94.275) (end 134.99687 94.275) (width 0.2) (layer "F.Cu") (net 11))
 (segment (start 138.6 74.5) (end 138.6 74.825927) (width 0.2) (layer "F.Cu") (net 11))
 (segment (start 131.99687 94.275) (end 133.49687 94.275) (width 0.2) (layer "F.Cu") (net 11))
 (segment (start 139.43437 94.9) (end 139.69887 94.9) (width 0.2) (layer "F.Cu") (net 11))
 (segment (start 138.6 74.825927) (end 139.150473 75.3764) (width 0.2) (layer "F.Cu") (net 11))
 (segment (start 139.43437 94.9) (end 139.43437 94.8375) (width 0.2) (layer "F.Cu") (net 11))
 (segment (start 139.69887 94.9) (end 139.99687 94.602) (width 0.2) (layer "F.Cu") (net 11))
 (via (at 139.99687 94.602) (size 0.6) (drill 0.3) (layers "F.Cu" "B.Cu") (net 11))
 (via (at 139.150473 75.3764) (size 0.6) (drill 0.3) (layers "F.Cu" "B.Cu") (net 11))
 (via (at 142.499 82.938026) (size 0.6) (drill 0.3) (layers "F.Cu" "B.Cu") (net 11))
 (via (at 143 74) (size 0.6) (drill 0.3) (layers "F.Cu" "B.Cu") (free yes) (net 11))
 (via (at 144 94.5) (size 0.6) (drill 0.3) (layers "F.Cu" "B.Cu") (free yes) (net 11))
 (via (at 129.5 94.5) (size 0.6) (drill 0.3) (layers "F.Cu" "B.Cu") (free yes) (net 11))
 (segment (start 138.49687 94.275) (end 139.99687 94.275) (width 0.2) (layer "B.Cu") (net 11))
 (segment (start 136.99687 94.275) (end 138.49687 94.275) (width 0.2) (layer "B.Cu") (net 11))
 (segment (start 141.7 87.29) (end 142.626 86.364) (width 0.2) (layer "B.Cu") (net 11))
 (segment (start 133.49687 94.275) (end 134.99687 94.275) (width 0.2) (layer "B.Cu") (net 11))
 (segment (start 142.626 86.364) (end 142.626 83.065026) (width 0.2) (layer "B.Cu") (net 11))
 (segment (start 142.626 83.065026) (end 142.499 82.938026) (width 0.2) (layer "B.Cu") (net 11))
 (segment (start 134.99687 94.275) (end 136.99687 94.275) (width 0.2) (layer "B.Cu") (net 11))
 (segment (start 140.1226 75.5) (end 141 75.5) (width 0.2) (layer "F.Cu") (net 12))
 (segment (start 137.55937 93.95) (end 136.22187 93.95) (width 0.2) (layer "F.Cu") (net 12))
 (segment (start 136.22187 93.95) (end 135.89061 93.61874) (width 0.2) (layer "F.Cu") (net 12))
 (segment (start 139.1 72.5) (end 139.1 74.4774) (width 0.2) (layer "F.Cu") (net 12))
 (segment (start 139.1 74.4774) (end 140.1226 75.5) (width 0.2) (layer "F.Cu") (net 12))
 (via (at 135.89061 93.61874) (size 0.6) (drill 0.3) (layers "F.Cu" "B.Cu") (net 12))
 (via (at 141 75.5) (size 0.6) (drill 0.3) (layers "F.Cu" "B.Cu") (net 12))
 (segment (start 135.89061 93.61874) (end 134.99687 92.725) (width 0.2) (layer "B.Cu") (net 12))
 (segment (start 130.074 90.75213) (end 131.99687 92.675) (width 0.2) (layer "B.Cu") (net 12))
 (segment (start 135.98535 93.524) (end 141.5 93.524) (width 0.2) (layer "B.Cu") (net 12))
 (segment (start 143.5 91.524) (end 143.5 78) (width 0.2) (layer "B.Cu") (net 12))
 (segment (start 141.5 93.524) (end 143.5 91.524) (width 0.2) (layer "B.Cu") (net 12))
 (segment (start 131.99687 92.675) (end 133.44687 92.675) (width 0.2) (layer "B.Cu") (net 12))
 (segment (start 133.49687 92.725) (end 134.99687 92.725) (width 0.2) (layer "B.Cu") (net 12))
 (segment (start 130.074 87.326) (end 130.074 90.75213) (width 0.2) (layer "B.Cu") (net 12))
 (segment (start 133.44687 92.675) (end 133.49687 92.725) (width 0.2) (layer "B.Cu") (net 12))
 (segment (start 143.5 78) (end 141 75.5) (width 0.2) (layer "B.Cu") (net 12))
 (segment (start 131 86.4) (end 130.074 87.326) (width 0.2) (layer "B.Cu") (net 12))
 (segment (start 135.89061 93.61874) (end 135.98535 93.524) (width 0.2) (layer "B.Cu") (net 12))
 (segment (start 131.99687 92.675) (end 131.902308 92.675) (width 0.2) (layer "B.Cu") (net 12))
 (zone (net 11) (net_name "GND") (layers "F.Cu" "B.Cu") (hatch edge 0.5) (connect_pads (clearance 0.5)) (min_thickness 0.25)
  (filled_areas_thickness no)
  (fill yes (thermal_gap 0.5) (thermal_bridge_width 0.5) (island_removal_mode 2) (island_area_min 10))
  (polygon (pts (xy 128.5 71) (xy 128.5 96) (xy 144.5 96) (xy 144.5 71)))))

